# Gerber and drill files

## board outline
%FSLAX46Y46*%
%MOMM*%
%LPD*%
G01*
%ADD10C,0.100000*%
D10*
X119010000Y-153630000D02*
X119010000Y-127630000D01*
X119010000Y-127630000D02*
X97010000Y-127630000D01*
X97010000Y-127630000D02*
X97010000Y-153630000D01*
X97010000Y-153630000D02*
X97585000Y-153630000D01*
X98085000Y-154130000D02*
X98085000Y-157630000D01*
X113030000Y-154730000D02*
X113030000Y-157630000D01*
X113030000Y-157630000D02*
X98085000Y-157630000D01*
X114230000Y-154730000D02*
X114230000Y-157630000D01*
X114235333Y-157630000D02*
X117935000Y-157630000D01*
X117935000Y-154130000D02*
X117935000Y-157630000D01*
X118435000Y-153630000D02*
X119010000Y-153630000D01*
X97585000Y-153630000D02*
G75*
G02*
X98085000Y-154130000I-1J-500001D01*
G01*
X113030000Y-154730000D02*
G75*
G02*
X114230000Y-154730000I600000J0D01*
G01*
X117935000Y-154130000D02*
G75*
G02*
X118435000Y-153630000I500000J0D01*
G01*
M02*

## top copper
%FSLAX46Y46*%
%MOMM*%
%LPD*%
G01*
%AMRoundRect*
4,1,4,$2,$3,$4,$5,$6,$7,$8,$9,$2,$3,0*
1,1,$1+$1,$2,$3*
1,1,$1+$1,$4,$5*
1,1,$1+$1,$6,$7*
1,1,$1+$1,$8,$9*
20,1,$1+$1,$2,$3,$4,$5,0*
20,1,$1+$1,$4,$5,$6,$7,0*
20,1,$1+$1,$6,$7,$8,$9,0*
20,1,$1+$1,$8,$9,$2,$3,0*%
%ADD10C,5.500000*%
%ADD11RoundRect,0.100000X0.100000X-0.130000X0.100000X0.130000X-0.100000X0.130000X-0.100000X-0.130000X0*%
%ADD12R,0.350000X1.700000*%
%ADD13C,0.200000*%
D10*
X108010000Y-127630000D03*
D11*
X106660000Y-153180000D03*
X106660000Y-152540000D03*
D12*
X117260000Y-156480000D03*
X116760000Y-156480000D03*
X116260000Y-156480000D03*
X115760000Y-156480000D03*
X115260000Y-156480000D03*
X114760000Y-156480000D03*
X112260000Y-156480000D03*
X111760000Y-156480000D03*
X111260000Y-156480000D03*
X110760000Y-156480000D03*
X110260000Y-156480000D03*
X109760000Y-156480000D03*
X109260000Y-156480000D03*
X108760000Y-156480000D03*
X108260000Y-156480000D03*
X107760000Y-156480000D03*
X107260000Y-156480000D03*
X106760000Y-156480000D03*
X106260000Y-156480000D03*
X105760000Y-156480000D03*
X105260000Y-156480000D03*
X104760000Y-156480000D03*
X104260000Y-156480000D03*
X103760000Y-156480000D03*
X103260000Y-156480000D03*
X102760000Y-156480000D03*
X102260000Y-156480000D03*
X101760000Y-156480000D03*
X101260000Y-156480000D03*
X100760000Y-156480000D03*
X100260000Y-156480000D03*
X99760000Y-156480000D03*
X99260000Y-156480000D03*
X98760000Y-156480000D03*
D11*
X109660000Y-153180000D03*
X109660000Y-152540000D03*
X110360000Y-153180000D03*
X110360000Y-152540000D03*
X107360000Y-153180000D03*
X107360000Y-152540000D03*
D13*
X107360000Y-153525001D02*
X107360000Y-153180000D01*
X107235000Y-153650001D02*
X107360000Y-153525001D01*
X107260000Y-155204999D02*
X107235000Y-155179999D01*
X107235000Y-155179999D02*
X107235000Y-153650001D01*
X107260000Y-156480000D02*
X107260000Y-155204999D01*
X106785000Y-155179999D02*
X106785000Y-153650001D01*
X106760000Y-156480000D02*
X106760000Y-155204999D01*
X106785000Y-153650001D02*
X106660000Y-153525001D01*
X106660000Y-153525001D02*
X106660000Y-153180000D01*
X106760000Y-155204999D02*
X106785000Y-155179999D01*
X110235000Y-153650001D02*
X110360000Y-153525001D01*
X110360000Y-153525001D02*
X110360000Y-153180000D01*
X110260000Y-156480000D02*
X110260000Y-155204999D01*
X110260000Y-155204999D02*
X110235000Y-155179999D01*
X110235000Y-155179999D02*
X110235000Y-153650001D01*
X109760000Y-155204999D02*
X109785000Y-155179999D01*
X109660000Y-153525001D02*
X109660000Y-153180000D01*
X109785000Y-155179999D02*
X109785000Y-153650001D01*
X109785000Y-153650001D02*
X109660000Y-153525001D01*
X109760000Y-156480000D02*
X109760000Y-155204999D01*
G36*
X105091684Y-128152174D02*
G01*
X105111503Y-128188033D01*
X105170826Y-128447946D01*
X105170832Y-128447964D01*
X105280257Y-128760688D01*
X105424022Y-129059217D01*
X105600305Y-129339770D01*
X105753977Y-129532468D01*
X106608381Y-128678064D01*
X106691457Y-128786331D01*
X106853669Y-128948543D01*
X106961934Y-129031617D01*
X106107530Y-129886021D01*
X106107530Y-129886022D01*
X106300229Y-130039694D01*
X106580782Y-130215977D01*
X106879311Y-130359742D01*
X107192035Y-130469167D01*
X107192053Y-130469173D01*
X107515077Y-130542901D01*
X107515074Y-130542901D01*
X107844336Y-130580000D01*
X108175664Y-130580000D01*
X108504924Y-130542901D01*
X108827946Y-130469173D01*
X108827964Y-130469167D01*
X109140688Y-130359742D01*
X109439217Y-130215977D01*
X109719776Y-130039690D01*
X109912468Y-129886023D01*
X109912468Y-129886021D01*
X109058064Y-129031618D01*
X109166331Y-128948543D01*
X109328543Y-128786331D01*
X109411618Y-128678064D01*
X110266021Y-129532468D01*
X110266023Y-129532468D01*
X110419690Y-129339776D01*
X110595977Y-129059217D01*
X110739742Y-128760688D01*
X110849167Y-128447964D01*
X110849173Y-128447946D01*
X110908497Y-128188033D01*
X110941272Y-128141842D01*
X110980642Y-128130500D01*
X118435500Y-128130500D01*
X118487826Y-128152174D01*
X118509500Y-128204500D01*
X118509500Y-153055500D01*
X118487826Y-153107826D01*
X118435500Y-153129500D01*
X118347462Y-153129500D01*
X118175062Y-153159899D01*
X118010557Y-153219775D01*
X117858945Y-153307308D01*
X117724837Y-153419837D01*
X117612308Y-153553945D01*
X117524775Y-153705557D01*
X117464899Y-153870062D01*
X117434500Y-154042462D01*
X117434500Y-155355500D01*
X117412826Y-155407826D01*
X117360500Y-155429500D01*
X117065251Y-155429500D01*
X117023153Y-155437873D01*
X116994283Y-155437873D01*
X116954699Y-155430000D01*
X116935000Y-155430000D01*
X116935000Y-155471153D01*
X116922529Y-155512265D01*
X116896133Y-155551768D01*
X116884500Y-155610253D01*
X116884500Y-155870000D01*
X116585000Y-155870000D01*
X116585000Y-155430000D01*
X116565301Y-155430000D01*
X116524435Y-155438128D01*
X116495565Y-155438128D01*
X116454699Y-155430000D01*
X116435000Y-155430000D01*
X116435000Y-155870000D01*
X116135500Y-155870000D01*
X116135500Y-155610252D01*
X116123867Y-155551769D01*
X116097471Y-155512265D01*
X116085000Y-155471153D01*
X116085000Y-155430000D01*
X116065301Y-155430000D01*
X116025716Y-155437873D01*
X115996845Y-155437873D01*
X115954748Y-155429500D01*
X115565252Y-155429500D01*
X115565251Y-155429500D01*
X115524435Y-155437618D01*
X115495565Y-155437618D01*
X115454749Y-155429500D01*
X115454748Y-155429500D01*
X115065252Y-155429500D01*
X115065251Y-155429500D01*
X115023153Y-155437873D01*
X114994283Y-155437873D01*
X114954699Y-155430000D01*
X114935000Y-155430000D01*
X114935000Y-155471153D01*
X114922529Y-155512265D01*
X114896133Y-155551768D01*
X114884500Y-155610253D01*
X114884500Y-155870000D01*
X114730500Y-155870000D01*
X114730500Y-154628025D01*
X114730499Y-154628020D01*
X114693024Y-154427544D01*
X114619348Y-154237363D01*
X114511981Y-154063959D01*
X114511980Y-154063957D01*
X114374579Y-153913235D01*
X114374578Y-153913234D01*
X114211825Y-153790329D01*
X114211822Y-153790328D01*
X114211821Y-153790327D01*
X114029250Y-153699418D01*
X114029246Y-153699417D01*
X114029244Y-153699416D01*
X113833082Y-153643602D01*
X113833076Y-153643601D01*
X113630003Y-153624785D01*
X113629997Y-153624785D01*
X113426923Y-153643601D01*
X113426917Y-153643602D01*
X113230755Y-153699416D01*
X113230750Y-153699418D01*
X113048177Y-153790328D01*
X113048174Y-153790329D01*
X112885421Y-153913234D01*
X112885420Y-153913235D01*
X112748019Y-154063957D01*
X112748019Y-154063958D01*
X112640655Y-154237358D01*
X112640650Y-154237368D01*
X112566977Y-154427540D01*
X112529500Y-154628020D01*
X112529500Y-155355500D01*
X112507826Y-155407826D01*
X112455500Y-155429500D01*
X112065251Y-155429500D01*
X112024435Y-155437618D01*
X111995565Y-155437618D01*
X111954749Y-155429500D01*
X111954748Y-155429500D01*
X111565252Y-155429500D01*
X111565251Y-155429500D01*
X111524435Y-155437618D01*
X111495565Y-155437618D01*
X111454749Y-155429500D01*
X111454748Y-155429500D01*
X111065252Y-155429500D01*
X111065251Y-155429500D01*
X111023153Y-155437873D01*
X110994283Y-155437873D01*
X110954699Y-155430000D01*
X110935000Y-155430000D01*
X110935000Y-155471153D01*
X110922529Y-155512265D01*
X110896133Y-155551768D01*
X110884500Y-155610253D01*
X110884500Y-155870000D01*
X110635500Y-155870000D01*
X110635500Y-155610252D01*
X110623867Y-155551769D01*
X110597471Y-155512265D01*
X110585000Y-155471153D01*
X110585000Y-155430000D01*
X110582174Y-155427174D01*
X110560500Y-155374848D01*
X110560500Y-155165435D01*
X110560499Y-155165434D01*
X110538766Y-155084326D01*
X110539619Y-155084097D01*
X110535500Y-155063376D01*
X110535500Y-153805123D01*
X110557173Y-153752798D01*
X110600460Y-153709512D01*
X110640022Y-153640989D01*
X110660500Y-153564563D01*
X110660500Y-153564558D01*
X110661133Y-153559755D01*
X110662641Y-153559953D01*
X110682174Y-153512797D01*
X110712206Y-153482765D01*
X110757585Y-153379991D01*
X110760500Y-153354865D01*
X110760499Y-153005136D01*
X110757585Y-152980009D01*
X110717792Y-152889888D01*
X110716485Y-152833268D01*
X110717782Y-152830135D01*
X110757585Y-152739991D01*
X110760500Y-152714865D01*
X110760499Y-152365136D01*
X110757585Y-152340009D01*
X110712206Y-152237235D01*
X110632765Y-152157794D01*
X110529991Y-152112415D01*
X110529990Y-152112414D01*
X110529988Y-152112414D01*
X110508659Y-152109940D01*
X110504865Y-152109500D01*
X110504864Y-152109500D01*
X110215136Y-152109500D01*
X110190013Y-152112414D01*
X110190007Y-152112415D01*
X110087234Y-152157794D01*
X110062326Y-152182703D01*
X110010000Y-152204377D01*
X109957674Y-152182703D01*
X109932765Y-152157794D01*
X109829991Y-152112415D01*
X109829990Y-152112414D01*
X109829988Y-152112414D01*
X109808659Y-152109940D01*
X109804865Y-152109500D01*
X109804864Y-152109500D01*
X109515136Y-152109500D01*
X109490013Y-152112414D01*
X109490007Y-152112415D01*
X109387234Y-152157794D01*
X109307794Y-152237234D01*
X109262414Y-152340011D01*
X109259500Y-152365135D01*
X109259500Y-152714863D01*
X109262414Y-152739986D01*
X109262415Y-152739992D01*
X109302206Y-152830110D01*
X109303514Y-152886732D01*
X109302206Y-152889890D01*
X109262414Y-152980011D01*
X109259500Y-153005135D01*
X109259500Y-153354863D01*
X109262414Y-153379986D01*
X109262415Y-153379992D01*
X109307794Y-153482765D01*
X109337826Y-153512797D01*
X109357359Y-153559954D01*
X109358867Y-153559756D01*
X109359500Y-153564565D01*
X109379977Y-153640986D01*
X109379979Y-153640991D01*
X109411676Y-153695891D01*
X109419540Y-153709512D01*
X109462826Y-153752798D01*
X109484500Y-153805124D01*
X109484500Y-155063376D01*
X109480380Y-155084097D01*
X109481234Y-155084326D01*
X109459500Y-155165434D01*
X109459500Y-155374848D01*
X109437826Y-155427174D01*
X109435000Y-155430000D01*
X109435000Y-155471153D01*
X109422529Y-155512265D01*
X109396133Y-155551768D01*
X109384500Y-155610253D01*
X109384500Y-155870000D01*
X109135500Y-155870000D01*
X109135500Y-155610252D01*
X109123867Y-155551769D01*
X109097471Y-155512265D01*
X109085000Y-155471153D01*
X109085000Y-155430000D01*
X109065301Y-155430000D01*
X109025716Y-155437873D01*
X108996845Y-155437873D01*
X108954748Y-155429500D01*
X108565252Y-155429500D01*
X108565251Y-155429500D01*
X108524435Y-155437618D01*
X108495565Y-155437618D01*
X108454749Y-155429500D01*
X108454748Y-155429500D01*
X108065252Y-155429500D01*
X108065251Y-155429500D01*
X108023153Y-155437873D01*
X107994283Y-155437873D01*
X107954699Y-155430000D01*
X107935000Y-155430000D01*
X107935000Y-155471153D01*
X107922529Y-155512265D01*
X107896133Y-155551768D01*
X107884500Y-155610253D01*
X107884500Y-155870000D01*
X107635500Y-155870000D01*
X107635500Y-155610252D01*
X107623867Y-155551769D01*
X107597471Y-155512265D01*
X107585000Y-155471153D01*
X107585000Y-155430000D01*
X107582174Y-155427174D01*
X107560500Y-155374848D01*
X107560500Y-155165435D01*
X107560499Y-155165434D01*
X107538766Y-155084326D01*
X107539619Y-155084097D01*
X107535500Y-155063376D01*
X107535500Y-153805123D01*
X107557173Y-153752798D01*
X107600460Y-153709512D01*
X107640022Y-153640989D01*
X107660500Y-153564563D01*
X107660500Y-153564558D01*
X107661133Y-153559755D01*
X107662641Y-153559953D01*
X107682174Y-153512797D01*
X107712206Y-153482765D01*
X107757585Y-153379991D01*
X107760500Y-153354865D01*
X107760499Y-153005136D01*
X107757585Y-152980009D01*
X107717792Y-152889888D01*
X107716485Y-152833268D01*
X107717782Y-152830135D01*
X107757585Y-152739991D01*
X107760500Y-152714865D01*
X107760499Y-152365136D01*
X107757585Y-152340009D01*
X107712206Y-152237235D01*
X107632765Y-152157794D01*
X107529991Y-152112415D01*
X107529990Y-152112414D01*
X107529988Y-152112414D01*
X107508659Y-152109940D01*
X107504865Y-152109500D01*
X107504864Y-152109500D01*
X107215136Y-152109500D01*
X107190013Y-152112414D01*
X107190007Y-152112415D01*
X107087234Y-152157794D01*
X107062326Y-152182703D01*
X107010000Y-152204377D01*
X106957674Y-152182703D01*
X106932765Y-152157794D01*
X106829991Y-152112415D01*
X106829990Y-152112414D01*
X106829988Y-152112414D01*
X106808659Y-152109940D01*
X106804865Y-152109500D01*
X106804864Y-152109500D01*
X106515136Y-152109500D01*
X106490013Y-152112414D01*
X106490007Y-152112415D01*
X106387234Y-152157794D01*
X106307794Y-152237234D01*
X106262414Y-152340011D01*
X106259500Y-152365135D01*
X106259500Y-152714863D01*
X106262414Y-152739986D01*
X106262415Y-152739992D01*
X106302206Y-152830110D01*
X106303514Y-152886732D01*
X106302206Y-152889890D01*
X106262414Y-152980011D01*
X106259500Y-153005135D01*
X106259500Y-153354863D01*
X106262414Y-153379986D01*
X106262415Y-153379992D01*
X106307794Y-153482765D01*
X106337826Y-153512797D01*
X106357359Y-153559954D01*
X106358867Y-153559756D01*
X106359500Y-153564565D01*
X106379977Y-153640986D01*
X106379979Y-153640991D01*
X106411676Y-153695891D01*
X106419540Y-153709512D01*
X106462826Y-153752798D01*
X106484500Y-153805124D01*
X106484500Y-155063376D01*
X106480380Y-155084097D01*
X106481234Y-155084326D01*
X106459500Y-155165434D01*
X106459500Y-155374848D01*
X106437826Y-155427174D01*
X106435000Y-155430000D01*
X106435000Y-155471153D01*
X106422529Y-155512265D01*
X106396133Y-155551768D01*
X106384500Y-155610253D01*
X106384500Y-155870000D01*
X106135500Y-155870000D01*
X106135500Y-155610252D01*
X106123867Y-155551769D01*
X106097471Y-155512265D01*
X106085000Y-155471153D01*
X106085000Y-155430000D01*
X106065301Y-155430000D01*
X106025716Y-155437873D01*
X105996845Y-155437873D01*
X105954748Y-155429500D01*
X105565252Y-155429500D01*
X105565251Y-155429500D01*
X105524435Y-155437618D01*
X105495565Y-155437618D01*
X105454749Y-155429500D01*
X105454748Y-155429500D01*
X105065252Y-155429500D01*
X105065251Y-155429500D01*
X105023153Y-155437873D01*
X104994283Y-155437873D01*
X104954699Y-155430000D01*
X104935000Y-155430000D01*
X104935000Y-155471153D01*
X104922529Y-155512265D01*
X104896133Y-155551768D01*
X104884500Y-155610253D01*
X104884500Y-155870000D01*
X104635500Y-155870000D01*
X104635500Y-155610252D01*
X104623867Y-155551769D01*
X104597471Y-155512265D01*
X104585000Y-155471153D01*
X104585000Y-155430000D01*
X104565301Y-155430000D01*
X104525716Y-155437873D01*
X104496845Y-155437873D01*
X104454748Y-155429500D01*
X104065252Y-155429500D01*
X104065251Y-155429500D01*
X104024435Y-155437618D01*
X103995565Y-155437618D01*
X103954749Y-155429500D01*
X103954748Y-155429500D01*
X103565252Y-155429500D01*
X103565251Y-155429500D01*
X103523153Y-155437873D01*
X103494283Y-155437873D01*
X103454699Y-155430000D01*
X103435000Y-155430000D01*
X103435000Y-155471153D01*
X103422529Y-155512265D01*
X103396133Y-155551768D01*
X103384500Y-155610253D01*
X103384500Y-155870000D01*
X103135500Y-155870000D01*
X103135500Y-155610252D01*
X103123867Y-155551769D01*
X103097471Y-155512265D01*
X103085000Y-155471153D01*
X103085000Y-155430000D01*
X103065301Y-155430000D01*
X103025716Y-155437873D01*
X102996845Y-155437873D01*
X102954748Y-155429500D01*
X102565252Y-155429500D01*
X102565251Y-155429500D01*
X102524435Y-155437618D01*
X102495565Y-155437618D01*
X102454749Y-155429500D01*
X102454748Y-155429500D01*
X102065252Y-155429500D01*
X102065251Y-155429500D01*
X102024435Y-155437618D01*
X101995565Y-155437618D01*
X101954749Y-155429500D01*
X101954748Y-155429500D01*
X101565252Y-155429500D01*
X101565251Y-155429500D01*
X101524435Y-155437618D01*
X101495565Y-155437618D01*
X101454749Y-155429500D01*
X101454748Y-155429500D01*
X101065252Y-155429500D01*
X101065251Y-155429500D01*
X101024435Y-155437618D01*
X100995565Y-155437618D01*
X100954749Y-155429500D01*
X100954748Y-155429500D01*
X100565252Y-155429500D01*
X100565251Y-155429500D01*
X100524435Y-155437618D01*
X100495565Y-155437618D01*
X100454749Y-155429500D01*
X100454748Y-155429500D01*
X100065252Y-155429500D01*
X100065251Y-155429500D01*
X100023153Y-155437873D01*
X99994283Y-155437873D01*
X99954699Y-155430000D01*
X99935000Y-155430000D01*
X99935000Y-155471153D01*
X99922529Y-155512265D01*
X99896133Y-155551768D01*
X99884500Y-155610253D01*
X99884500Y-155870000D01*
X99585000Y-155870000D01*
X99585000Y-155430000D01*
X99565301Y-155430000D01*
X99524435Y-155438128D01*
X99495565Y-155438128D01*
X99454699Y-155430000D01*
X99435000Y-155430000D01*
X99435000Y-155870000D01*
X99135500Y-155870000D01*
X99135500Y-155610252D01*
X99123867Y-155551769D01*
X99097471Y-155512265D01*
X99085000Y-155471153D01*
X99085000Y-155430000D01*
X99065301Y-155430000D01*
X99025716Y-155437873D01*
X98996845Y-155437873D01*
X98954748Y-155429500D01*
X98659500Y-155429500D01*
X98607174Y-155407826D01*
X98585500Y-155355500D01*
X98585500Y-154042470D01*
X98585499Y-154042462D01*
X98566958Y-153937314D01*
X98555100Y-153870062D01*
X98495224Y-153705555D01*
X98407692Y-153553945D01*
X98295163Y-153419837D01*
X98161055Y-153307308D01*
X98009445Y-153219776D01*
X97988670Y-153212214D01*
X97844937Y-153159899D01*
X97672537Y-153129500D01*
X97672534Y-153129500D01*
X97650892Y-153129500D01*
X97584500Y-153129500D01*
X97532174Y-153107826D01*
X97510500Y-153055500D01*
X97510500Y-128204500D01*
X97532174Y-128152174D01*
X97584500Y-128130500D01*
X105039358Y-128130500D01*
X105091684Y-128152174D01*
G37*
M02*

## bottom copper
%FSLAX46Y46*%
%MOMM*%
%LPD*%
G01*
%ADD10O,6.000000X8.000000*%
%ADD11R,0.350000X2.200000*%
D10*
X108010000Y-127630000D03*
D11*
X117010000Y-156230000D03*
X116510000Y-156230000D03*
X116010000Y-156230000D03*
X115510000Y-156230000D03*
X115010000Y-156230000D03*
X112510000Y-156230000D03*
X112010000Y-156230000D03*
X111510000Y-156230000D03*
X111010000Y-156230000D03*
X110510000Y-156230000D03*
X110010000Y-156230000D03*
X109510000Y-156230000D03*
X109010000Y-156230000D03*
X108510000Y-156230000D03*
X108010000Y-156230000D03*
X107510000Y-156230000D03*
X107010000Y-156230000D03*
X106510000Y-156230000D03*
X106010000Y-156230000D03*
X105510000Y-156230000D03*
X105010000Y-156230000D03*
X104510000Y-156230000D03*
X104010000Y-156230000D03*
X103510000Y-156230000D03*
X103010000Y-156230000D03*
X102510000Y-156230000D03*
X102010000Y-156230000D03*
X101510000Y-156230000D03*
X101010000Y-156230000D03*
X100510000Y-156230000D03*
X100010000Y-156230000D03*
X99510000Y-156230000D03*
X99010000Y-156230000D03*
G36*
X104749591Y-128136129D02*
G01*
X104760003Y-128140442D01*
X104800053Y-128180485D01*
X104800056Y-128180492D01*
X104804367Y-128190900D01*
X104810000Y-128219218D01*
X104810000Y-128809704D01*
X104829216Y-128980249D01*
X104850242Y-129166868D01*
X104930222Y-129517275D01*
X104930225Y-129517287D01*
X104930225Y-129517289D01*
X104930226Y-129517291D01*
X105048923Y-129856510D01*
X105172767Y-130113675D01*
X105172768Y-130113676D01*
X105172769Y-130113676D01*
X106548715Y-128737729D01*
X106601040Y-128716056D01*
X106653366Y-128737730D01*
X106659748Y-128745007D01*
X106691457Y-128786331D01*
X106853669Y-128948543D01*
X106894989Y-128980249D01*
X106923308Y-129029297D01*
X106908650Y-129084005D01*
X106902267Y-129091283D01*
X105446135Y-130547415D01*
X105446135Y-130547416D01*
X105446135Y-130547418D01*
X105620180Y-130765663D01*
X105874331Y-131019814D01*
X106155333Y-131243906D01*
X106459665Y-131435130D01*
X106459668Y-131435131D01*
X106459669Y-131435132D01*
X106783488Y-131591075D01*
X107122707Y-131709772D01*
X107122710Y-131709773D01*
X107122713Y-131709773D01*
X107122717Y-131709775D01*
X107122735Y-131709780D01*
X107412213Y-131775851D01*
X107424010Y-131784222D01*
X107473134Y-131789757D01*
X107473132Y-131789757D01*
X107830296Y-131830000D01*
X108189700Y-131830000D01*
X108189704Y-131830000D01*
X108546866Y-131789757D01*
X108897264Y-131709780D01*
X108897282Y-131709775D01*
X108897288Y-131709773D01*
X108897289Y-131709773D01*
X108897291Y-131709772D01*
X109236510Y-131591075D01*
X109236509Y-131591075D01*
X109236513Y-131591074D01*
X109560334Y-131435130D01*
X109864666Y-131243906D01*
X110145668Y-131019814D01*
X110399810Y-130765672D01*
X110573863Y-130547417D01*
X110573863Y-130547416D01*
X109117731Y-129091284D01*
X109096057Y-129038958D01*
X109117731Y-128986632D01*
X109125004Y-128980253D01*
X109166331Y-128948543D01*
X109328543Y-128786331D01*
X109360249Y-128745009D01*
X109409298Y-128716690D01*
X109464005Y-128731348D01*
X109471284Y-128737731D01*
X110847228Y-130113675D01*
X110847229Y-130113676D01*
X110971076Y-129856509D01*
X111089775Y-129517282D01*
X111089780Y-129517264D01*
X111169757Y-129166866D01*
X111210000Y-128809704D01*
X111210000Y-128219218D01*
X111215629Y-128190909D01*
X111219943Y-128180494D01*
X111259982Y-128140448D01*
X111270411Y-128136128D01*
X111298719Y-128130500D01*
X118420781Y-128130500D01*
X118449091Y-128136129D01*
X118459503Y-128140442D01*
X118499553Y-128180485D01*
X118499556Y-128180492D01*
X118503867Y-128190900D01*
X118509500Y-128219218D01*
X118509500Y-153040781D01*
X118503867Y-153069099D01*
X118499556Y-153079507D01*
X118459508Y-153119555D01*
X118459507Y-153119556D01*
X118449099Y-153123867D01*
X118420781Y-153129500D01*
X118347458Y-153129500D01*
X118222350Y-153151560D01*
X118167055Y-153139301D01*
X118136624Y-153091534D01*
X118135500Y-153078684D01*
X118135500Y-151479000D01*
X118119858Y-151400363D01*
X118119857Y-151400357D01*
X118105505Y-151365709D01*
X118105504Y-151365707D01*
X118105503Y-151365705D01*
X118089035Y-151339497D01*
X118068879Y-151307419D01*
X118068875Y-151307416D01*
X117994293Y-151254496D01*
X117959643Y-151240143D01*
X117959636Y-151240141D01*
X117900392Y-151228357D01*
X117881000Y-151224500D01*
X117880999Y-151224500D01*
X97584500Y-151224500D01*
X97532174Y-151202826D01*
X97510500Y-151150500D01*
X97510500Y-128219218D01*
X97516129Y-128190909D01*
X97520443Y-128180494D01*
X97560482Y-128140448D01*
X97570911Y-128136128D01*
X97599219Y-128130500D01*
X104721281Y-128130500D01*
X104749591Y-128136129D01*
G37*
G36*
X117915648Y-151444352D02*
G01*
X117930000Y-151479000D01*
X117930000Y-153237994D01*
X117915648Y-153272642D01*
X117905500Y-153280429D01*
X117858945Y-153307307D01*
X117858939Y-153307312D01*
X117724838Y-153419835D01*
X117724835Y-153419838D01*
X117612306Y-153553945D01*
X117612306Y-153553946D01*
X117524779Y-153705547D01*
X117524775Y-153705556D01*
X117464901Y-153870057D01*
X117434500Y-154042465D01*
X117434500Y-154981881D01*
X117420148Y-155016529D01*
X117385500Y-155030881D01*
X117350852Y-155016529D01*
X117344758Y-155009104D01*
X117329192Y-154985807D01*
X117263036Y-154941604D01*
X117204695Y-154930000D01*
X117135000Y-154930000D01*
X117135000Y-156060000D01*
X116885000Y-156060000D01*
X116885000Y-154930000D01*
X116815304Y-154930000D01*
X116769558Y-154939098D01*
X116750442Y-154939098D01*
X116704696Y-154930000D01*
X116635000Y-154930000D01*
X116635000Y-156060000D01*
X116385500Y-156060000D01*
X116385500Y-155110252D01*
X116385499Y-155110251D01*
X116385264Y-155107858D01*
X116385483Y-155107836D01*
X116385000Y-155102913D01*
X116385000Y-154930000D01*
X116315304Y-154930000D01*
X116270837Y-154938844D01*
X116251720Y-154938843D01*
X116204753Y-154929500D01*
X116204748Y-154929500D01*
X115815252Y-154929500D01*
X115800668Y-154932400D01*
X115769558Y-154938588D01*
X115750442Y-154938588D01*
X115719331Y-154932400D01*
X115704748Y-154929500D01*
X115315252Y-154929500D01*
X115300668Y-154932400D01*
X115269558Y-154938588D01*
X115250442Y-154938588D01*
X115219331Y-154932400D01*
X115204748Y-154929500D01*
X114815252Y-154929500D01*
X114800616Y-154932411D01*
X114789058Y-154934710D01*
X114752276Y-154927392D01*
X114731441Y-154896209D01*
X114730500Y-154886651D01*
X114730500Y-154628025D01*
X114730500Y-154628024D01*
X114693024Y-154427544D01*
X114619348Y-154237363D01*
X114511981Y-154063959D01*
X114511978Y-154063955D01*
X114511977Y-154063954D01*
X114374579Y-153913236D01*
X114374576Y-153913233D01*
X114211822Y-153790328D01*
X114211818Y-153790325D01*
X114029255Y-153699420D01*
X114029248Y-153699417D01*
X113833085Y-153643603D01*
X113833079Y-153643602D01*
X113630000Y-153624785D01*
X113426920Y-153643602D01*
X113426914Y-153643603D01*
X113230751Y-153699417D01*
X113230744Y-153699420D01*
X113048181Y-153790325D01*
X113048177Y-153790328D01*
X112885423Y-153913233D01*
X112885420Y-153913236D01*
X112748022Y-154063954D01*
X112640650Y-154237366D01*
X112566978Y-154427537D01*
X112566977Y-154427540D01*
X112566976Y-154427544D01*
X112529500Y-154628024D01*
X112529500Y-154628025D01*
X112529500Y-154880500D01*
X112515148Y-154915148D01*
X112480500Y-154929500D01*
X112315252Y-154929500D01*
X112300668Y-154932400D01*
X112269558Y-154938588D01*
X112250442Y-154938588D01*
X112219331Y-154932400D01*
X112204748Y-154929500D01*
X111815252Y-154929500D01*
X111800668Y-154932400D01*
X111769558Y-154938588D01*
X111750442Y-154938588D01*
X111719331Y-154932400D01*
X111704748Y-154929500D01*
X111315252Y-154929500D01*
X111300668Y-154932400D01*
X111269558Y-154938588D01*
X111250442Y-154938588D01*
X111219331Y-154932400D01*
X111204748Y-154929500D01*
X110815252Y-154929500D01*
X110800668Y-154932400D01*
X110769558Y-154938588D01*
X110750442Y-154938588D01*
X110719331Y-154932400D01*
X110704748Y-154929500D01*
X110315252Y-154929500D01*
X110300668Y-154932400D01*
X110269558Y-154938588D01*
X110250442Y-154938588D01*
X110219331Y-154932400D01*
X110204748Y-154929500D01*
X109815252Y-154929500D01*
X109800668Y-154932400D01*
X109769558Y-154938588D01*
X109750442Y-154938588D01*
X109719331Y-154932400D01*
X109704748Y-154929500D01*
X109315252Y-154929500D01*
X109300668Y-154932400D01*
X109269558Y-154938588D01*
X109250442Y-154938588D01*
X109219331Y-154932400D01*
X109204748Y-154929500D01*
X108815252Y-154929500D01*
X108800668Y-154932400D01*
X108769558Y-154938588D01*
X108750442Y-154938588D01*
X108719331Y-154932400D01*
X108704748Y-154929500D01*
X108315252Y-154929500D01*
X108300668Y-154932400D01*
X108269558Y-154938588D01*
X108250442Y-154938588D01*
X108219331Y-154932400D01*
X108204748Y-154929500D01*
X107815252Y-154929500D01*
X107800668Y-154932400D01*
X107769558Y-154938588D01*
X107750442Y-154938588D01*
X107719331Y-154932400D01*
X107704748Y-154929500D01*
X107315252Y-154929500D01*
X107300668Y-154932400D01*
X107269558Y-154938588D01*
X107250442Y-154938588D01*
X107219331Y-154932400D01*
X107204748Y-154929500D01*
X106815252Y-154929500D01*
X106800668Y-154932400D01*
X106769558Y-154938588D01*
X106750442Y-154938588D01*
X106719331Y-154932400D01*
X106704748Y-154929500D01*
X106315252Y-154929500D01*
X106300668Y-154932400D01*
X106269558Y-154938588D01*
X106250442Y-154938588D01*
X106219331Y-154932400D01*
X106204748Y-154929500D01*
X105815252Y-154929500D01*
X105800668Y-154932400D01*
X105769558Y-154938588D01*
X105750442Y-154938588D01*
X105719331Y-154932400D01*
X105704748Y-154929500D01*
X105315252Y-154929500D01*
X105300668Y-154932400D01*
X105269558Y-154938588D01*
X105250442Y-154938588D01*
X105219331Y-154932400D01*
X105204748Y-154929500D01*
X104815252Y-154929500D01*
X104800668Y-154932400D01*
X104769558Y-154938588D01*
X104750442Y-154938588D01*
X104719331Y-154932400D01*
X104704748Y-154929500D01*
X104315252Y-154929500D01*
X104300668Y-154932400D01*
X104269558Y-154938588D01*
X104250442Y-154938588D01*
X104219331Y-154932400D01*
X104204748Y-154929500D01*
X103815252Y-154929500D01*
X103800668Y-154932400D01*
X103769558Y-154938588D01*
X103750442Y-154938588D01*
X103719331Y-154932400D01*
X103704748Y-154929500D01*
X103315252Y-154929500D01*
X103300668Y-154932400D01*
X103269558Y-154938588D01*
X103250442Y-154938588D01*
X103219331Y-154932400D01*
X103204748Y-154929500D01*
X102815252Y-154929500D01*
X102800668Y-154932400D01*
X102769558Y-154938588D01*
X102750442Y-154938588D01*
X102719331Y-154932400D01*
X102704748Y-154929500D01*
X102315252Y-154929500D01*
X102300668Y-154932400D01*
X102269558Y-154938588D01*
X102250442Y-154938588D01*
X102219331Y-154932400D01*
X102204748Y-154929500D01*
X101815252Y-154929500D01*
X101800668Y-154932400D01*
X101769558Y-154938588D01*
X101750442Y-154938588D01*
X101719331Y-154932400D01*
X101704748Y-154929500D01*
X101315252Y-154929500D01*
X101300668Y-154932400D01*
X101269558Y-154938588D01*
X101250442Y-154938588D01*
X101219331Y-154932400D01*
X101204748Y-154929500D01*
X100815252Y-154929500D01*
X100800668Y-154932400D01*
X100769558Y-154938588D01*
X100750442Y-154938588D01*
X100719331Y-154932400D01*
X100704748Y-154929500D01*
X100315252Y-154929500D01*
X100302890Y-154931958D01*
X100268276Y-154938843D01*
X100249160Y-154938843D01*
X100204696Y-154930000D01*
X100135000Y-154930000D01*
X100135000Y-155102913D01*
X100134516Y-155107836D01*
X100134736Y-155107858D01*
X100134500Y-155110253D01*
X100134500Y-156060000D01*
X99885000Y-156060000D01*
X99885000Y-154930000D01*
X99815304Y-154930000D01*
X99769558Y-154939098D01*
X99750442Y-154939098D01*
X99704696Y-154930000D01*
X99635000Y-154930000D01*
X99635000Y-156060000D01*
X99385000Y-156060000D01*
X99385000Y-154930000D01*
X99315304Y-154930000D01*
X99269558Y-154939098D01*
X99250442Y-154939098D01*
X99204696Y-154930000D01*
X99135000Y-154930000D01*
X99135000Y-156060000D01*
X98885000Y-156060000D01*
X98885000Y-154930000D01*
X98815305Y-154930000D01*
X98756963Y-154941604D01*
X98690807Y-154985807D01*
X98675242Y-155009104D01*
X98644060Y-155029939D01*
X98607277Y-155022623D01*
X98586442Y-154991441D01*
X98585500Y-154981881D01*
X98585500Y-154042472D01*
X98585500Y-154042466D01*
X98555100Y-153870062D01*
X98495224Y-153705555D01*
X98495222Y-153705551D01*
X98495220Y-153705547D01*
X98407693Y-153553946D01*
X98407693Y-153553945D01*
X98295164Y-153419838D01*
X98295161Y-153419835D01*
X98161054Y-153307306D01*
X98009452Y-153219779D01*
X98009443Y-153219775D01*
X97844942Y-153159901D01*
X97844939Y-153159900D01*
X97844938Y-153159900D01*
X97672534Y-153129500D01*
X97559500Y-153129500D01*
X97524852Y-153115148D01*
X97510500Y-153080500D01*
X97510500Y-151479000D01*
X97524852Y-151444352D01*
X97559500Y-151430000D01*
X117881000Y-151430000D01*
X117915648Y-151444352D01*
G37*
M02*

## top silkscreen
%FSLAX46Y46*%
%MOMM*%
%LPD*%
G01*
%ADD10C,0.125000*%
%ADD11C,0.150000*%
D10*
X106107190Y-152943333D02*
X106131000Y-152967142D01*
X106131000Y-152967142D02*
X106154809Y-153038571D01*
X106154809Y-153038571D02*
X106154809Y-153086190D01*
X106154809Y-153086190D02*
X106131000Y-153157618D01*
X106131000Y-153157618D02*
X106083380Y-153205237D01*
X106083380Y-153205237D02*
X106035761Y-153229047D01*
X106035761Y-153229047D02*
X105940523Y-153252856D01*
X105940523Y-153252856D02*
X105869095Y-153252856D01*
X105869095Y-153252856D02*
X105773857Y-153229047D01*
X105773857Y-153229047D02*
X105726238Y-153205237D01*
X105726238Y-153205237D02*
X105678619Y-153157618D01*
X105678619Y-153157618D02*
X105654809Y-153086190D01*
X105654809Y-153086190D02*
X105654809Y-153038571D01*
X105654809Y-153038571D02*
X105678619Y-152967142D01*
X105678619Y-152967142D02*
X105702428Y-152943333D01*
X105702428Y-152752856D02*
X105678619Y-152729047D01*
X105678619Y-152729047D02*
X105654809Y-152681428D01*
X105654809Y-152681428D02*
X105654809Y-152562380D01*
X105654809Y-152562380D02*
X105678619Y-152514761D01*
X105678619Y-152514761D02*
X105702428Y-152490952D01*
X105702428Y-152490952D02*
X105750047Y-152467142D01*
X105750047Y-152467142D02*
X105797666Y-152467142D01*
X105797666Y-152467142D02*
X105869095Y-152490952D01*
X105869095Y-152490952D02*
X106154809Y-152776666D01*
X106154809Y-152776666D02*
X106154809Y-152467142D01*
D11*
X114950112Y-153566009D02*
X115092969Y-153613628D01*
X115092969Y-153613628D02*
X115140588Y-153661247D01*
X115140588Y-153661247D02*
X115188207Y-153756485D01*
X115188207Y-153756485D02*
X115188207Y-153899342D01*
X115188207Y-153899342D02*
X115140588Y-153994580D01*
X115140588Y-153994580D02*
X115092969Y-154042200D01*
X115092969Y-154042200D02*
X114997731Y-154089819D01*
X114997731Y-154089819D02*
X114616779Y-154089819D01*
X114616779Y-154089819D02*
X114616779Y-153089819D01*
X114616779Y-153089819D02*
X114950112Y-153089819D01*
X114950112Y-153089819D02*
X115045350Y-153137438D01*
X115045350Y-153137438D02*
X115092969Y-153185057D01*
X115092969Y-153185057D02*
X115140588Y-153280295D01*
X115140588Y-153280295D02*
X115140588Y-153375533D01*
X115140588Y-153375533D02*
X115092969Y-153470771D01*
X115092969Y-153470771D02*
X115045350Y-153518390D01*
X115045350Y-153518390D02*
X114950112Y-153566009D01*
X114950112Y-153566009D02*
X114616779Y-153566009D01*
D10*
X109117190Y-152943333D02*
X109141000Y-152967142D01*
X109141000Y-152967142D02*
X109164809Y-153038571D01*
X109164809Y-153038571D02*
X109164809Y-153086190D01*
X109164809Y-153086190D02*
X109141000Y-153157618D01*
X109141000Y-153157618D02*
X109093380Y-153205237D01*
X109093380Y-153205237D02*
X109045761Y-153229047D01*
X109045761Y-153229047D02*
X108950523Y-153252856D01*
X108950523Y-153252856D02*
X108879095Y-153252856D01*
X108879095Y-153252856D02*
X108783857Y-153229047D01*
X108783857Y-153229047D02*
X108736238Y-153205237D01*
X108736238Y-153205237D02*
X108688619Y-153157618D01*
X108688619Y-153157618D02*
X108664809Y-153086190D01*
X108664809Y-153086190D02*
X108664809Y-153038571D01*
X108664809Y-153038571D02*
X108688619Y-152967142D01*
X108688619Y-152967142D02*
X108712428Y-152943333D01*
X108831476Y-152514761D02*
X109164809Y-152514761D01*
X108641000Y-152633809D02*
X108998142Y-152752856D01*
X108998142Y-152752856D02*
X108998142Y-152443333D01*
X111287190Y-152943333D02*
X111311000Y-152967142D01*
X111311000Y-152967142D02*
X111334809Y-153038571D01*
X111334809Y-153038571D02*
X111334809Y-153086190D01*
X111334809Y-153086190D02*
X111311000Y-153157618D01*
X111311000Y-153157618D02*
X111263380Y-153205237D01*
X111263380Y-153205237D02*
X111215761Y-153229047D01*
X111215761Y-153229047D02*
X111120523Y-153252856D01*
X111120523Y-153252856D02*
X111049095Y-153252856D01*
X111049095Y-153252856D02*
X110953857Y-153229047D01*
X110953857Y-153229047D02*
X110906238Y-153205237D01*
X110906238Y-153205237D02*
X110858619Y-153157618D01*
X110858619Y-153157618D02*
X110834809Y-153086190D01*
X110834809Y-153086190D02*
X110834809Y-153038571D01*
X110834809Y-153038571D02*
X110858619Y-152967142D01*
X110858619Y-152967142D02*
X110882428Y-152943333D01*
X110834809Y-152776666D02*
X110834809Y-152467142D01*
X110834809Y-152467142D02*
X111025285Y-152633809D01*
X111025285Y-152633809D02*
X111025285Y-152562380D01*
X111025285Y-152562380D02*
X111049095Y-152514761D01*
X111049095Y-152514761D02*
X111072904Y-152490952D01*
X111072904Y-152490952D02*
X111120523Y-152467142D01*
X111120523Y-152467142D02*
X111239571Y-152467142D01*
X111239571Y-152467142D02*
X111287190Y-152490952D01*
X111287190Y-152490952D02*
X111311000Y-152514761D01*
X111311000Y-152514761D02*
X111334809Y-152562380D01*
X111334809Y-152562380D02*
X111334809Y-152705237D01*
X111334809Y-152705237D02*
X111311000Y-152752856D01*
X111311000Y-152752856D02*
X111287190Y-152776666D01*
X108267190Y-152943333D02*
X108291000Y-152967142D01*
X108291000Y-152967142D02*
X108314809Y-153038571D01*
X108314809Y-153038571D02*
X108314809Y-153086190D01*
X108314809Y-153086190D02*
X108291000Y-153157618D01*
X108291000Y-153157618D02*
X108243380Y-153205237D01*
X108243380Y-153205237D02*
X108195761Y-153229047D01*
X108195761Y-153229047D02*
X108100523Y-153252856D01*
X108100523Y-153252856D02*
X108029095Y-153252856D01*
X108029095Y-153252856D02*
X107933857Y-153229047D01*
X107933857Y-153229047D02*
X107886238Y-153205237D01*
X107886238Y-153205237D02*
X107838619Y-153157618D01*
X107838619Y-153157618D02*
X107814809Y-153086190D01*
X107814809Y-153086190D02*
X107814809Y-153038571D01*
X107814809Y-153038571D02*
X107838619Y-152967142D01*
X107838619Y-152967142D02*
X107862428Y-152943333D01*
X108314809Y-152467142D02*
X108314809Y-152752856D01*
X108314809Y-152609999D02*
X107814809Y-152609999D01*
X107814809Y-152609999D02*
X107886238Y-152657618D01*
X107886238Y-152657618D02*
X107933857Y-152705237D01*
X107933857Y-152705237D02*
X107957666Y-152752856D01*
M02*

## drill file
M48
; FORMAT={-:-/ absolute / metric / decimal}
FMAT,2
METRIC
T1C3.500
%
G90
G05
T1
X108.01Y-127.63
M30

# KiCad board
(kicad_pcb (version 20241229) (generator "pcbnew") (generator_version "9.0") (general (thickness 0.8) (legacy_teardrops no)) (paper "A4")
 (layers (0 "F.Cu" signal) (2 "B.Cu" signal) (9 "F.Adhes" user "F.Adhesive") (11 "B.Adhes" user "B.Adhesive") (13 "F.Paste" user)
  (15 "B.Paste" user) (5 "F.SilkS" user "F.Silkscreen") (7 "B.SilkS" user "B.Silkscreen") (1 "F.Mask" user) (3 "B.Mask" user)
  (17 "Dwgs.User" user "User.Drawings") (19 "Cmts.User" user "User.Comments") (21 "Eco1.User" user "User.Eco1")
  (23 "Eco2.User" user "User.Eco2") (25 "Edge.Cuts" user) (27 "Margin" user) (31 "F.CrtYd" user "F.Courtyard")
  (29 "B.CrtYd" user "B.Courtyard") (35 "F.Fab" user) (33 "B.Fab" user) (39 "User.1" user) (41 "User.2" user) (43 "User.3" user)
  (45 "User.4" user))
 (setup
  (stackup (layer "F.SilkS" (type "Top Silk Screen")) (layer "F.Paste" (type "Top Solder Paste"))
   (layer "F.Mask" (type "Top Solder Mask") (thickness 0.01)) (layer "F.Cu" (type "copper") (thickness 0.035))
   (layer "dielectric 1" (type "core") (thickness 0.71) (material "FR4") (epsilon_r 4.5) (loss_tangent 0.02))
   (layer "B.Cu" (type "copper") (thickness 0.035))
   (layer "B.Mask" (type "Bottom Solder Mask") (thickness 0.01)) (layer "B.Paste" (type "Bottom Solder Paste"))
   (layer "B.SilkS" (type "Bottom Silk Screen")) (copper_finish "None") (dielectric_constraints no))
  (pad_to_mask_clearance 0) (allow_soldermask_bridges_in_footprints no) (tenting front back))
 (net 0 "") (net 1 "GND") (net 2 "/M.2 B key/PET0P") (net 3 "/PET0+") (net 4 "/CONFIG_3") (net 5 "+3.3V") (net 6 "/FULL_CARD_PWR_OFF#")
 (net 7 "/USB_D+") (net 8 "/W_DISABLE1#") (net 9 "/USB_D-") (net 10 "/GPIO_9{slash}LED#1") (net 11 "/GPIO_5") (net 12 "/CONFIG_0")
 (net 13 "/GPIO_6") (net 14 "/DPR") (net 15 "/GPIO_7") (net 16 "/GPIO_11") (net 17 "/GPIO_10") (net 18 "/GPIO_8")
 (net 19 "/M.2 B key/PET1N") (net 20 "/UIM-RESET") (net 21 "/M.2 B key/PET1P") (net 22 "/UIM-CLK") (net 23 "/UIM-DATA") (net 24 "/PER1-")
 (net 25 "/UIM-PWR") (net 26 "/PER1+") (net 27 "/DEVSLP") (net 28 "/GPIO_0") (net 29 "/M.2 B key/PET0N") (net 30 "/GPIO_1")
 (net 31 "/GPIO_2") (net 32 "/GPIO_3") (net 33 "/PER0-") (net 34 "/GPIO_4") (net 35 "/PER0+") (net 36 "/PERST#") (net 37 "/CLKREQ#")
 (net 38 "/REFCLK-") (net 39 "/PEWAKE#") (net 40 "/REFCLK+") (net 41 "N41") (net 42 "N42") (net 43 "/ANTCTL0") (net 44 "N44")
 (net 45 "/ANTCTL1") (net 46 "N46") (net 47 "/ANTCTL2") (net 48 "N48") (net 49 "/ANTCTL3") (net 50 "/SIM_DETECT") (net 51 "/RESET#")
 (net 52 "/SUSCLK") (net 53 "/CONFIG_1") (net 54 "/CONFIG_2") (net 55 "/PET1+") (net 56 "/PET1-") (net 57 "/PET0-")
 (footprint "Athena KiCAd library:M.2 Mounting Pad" (layer "F.Cu") (at 108.01 127.63)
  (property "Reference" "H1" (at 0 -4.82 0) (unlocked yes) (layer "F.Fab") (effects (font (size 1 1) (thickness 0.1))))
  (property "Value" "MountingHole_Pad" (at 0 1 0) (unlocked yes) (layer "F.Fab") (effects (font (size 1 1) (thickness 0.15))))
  (pad "1" thru_hole circle (at 0 0) (size 5.5 5.5) (drill 3.5) (layers "*.Cu" "*.Mask") (remove_unused_layers no) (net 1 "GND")
   (padstack (mode front_inner_back)
    (layer "Inner" (shape circle) (size 5.5 5.5) (zone_connect -1))
    (layer "B.Cu" (shape oval) (size 6 8) (thermal_bridge_angle 45) (zone_connect -1)))))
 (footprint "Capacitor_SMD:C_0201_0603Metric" (layer "F.Cu") (at 106.66 152.86 90)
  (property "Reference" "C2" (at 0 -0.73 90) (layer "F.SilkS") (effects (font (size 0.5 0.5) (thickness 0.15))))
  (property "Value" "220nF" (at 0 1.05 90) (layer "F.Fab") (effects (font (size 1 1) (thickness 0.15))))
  (pad "" smd roundrect (at -0.345 0 90) (size 0.318 0.36) (layers "F.Paste") (roundrect_rratio 0.25))
  (pad "" smd roundrect (at 0.345 0 90) (size 0.318 0.36) (layers "F.Paste") (roundrect_rratio 0.25))
  (pad "1" smd roundrect (at -0.32 0 90) (size 0.46 0.4) (layers "F.Cu" "F.Mask") (roundrect_rratio 0.25) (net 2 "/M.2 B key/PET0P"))
  (pad "2" smd roundrect (at 0.32 0 90) (size 0.46 0.4) (layers "F.Cu" "F.Mask") (roundrect_rratio 0.25) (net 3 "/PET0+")))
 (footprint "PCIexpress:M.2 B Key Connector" (layer "F.Cu") (at 108.01 156.52)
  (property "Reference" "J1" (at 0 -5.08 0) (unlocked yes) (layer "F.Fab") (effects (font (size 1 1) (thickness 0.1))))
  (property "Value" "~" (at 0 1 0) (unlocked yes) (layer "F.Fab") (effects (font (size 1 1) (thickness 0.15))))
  (fp_line (start -11 -2.89) (end -10.425 -2.89) (stroke (width 0.1) (type default)) (layer "Edge.Cuts"))
  (fp_line (start -9.925 -2.39) (end -9.925 1.11) (stroke (width 0.1) (type default)) (layer "Edge.Cuts"))
  (fp_line (start 5.02 -1.79) (end 5.02 1.11) (stroke (width 0.1) (type default)) (layer "Edge.Cuts"))
  (fp_line (start 5.02 1.11) (end -9.925 1.11) (stroke (width 0.1) (type default)) (layer "Edge.Cuts"))
  (fp_line (start 6.22 -1.79) (end 6.22 1.11) (stroke (width 0.1) (type default)) (layer "Edge.Cuts"))
  (fp_line (start 6.225333 1.11) (end 9.925 1.11) (stroke (width 0.1) (type default)) (layer "Edge.Cuts"))
  (fp_line (start 9.925 -2.39) (end 9.925 1.11) (stroke (width 0.1) (type default)) (layer "Edge.Cuts"))
  (fp_line (start 10.425 -2.89) (end 11 -2.89) (stroke (width 0.1) (type default)) (layer "Edge.Cuts"))
  (fp_arc (start -10.425 -2.89) (mid -10.071447 -2.743553) (end -9.925 -2.39) (stroke (width 0.1) (type default)) (layer "Edge.Cuts"))
  (fp_arc (start 5.02 -1.79) (mid 5.62 -2.39) (end 6.22 -1.79) (stroke (width 0.1) (type default)) (layer "Edge.Cuts"))
  (fp_arc (start 9.925 -2.39) (mid 10.071447 -2.743553) (end 10.425 -2.89) (stroke (width 0.1) (type default)) (layer "Edge.Cuts"))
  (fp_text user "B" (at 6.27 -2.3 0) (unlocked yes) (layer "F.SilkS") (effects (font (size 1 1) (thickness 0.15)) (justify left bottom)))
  (pad "1" smd rect (at 9.25 -0.04 180) (size 0.35 1.7) (layers "F.Cu") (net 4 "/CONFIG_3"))
  (pad "2" smd rect (at 9 -0.29 180) (size 0.35 2.2) (layers "B.Cu") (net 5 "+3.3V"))
  (pad "3" smd rect (at 8.75 -0.04 180) (size 0.35 1.7) (layers "F.Cu") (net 1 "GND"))
  (pad "4" smd rect (at 8.5 -0.29 180) (size 0.35 2.2) (layers "B.Cu") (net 5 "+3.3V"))
  (pad "5" smd rect (at 8.25 -0.04 180) (size 0.35 1.7) (layers "F.Cu") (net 1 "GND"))
  (pad "6" smd rect (at 8 -0.29 180) (size 0.35 2.2) (layers "B.Cu") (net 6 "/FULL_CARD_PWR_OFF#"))
  (pad "7" smd rect (at 7.75 -0.04 180) (size 0.35 1.7) (layers "F.Cu") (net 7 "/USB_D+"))
  (pad "8" smd rect (at 7.5 -0.29 180) (size 0.35 2.2) (layers "B.Cu") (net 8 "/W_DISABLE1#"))
  (pad "9" smd rect (at 7.25 -0.04 180) (size 0.35 1.7) (layers "F.Cu") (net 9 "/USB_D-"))
  (pad "10" smd rect (at 7 -0.29 180) (size 0.35 2.2) (layers "B.Cu") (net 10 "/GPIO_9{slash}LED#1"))
  (pad "11" smd rect (at 6.75 -0.04 180) (size 0.35 1.7) (layers "F.Cu") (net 1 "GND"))
  (pad "20" smd rect (at 4.5 -0.29 180) (size 0.35 2.2) (layers "B.Cu") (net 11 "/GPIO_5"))
  (pad "21" smd rect (at 4.25 -0.04 180) (size 0.35 1.7) (layers "F.Cu") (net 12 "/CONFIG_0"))
  (pad "22" smd rect (at 4 -0.29 180) (size 0.35 2.2) (layers "B.Cu") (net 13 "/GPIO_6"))
  (pad "23" smd rect (at 3.75 -0.04 180) (size 0.35 1.7) (layers "F.Cu") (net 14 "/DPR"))
  (pad "24" smd rect (at 3.5 -0.29 180) (size 0.35 2.2) (layers "B.Cu") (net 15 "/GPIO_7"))
  (pad "25" smd rect (at 3.25 -0.04 180) (size 0.35 1.7) (layers "F.Cu") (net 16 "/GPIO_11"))
  (pad "26" smd rect (at 3 -0.29 180) (size 0.35 2.2) (layers "B.Cu") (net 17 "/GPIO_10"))
  (pad "27" smd rect (at 2.75 -0.04 180) (size 0.35 1.7) (layers "F.Cu") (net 1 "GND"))
  (pad "28" smd rect (at 2.5 -0.29 180) (size 0.35 2.2) (layers "B.Cu") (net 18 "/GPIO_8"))
  (pad "29" smd rect (at 2.25 -0.04 180) (size 0.35 1.7) (layers "F.Cu") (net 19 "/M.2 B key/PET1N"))
  (pad "30" smd rect (at 2 -0.29 180) (size 0.35 2.2) (layers "B.Cu") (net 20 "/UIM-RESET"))
  (pad "31" smd rect (at 1.75 -0.04 180) (size 0.35 1.7) (layers "F.Cu") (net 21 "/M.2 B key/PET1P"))
  (pad "32" smd rect (at 1.5 -0.29 180) (size 0.35 2.2) (layers "B.Cu") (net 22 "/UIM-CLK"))
  (pad "33" smd rect (at 1.25 -0.04 180) (size 0.35 1.7) (layers "F.Cu") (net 1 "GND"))
  (pad "34" smd rect (at 1 -0.29 180) (size 0.35 2.2) (layers "B.Cu") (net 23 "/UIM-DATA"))
  (pad "35" smd rect (at 0.75 -0.04 180) (size 0.35 1.7) (layers "F.Cu") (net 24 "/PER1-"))
  (pad "36" smd rect (at 0.5 -0.29 180) (size 0.35 2.2) (layers "B.Cu") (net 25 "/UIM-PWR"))
  (pad "37" smd rect (at 0.25 -0.04 180) (size 0.35 1.7) (layers "F.Cu") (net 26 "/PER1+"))
  (pad "38" smd rect (at 0 -0.29 180) (size 0.35 2.2) (layers "B.Cu") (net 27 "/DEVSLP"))
  (pad "39" smd rect (at -0.25 -0.04 180) (size 0.35 1.7) (layers "F.Cu") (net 1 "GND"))
  (pad "40" smd rect (at -0.5 -0.29 180) (size 0.35 2.2) (layers "B.Cu") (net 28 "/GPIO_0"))
  (pad "41" smd rect (at -0.75 -0.04 180) (size 0.35 1.7) (layers "F.Cu") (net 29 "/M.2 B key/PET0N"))
  (pad "42" smd rect (at -1 -0.29 180) (size 0.35 2.2) (layers "B.Cu") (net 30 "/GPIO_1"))
  (pad "43" smd rect (at -1.25 -0.04 180) (size 0.35 1.7) (layers "F.Cu") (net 2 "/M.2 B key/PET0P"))
  (pad "44" smd rect (at -1.5 -0.29 180) (size 0.35 2.2) (layers "B.Cu") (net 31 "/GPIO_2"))
  (pad "45" smd rect (at -1.75 -0.04 180) (size 0.35 1.7) (layers "F.Cu") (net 1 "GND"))
  (pad "46" smd rect (at -2 -0.29 180) (size 0.35 2.2) (layers "B.Cu") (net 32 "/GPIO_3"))
  (pad "47" smd rect (at -2.25 -0.04 180) (size 0.35 1.7) (layers "F.Cu") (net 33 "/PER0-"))
  (pad "48" smd rect (at -2.5 -0.29 180) (size 0.35 2.2) (layers "B.Cu") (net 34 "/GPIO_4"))
  (pad "49" smd rect (at -2.75 -0.04 180) (size 0.35 1.7) (layers "F.Cu") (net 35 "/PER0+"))
  (pad "50" smd rect (at -3 -0.29 180) (size 0.35 2.2) (layers "B.Cu") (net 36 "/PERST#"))
  (pad "51" smd rect (at -3.25 -0.04 180) (size 0.35 1.7) (layers "F.Cu") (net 1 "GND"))
  (pad "52" smd rect (at -3.5 -0.29 180) (size 0.35 2.2) (layers "B.Cu") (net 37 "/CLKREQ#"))
  (pad "53" smd rect (at -3.75 -0.04 180) (size 0.35 1.7) (layers "F.Cu") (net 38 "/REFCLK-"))
  (pad "54" smd rect (at -4 -0.29 180) (size 0.35 2.2) (layers "B.Cu") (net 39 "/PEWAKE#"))
  (pad "55" smd rect (at -4.25 -0.04 180) (size 0.35 1.7) (layers "F.Cu") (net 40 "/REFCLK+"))
  (pad "56" smd rect (at -4.5 -0.29 180) (size 0.35 2.2) (layers "B.Cu") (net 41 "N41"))
  (pad "57" smd rect (at -4.75 -0.04 180) (size 0.35 1.7) (layers "F.Cu") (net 1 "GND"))
  (pad "58" smd rect (at -5 -0.29 180) (size 0.35 2.2) (layers "B.Cu") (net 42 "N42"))
  (pad "59" smd rect (at -5.25 -0.04 180) (size 0.35 1.7) (layers "F.Cu") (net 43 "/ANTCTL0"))
  (pad "60" smd rect (at -5.5 -0.29 180) (size 0.35 2.2) (layers "B.Cu") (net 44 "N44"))
  (pad "61" smd rect (at -5.75 -0.04 180) (size 0.35 1.7) (layers "F.Cu") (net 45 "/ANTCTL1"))
  (pad "62" smd rect (at -6 -0.29 180) (size 0.35 2.2) (layers "B.Cu") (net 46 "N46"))
  (pad "63" smd rect (at -6.25 -0.04 180) (size 0.35 1.7) (layers "F.Cu") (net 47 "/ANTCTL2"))
  (pad "64" smd rect (at -6.5 -0.29 180) (size 0.35 2.2) (layers "B.Cu") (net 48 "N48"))
  (pad "65" smd rect (at -6.75 -0.04 180) (size 0.35 1.7) (layers "F.Cu") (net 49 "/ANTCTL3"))
  (pad "66" smd rect (at -7 -0.29 180) (size 0.35 2.2) (layers "B.Cu") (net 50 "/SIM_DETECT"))
  (pad "67" smd rect (at -7.25 -0.04 180) (size 0.35 1.7) (layers "F.Cu") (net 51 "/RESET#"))
  (pad "68" smd rect (at -7.5 -0.29 180) (size 0.35 2.2) (layers "B.Cu") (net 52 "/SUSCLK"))
  (pad "69" smd rect (at -7.75 -0.04 180) (size 0.35 1.7) (layers "F.Cu") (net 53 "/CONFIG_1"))
  (pad "70" smd rect (at -8 -0.29 180) (size 0.35 2.2) (layers "B.Cu") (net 5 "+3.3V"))
  (pad "71" smd rect (at -8.25 -0.04 180) (size 0.35 1.7) (layers "F.Cu") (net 1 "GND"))
  (pad "72" smd rect (at -8.5 -0.29 180) (size 0.35 2.2) (layers "B.Cu") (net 5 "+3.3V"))
  (pad "73" smd rect (at -8.75 -0.04 180) (size 0.35 1.7) (layers "F.Cu") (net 1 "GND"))
  (pad "74" smd rect (at -9 -0.29 180) (size 0.35 2.2) (layers "B.Cu") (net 5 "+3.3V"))
  (pad "75" smd rect (at -9.25 -0.04 180) (size 0.35 1.7) (layers "F.Cu") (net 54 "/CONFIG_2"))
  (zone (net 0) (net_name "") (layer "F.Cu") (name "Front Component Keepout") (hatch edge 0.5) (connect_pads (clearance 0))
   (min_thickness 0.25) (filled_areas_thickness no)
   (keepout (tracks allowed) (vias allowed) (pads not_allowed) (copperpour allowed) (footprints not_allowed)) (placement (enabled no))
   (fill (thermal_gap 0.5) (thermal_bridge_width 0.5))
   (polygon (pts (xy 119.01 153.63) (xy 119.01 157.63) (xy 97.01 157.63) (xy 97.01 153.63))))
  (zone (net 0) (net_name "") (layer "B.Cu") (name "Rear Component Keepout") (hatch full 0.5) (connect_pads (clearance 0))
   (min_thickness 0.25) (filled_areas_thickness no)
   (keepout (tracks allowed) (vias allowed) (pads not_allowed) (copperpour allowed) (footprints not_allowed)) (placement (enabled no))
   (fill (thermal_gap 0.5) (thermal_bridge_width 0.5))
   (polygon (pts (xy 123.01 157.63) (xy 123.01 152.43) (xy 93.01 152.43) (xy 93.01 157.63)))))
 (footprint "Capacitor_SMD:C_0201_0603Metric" (layer "F.Cu") (at 109.66 152.86 90)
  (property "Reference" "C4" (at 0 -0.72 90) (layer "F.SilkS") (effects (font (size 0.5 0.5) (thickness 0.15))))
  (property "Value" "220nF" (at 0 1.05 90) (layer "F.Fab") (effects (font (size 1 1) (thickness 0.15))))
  (pad "" smd roundrect (at -0.345 0 90) (size 0.318 0.36) (layers "F.Paste") (roundrect_rratio 0.25))
  (pad "" smd roundrect (at 0.345 0 90) (size 0.318 0.36) (layers "F.Paste") (roundrect_rratio 0.25))
  (pad "1" smd roundrect (at -0.32 0 90) (size 0.46 0.4) (layers "F.Cu" "F.Mask") (roundrect_rratio 0.25) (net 21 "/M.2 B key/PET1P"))
  (pad "2" smd roundrect (at 0.32 0 90) (size 0.46 0.4) (layers "F.Cu" "F.Mask") (roundrect_rratio 0.25) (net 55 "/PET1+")))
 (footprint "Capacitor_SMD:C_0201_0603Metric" (layer "F.Cu") (at 110.36 152.86 90)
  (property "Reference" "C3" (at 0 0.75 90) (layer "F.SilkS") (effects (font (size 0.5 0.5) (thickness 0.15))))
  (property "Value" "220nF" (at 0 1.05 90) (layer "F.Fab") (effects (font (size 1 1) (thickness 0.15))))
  (pad "" smd roundrect (at -0.345 0 90) (size 0.318 0.36) (layers "F.Paste") (roundrect_rratio 0.25))
  (pad "" smd roundrect (at 0.345 0 90) (size 0.318 0.36) (layers "F.Paste") (roundrect_rratio 0.25))
  (pad "1" smd roundrect (at -0.32 0 90) (size 0.46 0.4) (layers "F.Cu" "F.Mask") (roundrect_rratio 0.25) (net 19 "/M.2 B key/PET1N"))
  (pad "2" smd roundrect (at 0.32 0 90) (size 0.46 0.4) (layers "F.Cu" "F.Mask") (roundrect_rratio 0.25) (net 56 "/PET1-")))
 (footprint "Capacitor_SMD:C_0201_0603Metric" (layer "F.Cu") (at 107.36 152.86 90)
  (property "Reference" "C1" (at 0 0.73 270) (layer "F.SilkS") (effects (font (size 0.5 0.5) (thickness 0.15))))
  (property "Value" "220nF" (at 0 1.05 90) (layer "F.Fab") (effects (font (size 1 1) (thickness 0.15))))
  (pad "" smd roundrect (at -0.345 0 90) (size 0.318 0.36) (layers "F.Paste") (roundrect_rratio 0.25))
  (pad "" smd roundrect (at 0.345 0 90) (size 0.318 0.36) (layers "F.Paste") (roundrect_rratio 0.25))
  (pad "1" smd roundrect (at -0.32 0 90) (size 0.46 0.4) (layers "F.Cu" "F.Mask") (roundrect_rratio 0.25) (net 29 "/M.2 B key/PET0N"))
  (pad "2" smd roundrect (at 0.32 0 90) (size 0.46 0.4) (layers "F.Cu" "F.Mask") (roundrect_rratio 0.25) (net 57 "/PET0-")))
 (gr_line (start 119.01 153.63) (end 119.01 127.63) (stroke (width 0.1) (type default)) (layer "Edge.Cuts"))
 (gr_line (start 119.01 127.63) (end 97.01 127.63) (stroke (width 0.1) (type default)) (layer "Edge.Cuts"))
 (gr_line (start 97.01 127.63) (end 97.01 153.63) (stroke (width 0.1) (type default)) (layer "Edge.Cuts"))
 (segment (start 107.36 153.525001) (end 107.36 153.18) (width 0.2) (layer "F.Cu") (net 29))
 (segment (start 107.235 153.650001) (end 107.36 153.525001) (width 0.2) (layer "F.Cu") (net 29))
 (segment (start 107.26 155.204999) (end 107.235 155.179999) (width 0.2) (layer "F.Cu") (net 29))
 (segment (start 107.235 155.179999) (end 107.235 153.650001) (width 0.2) (layer "F.Cu") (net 29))
 (segment (start 107.26 156.48) (end 107.26 155.204999) (width 0.2) (layer "F.Cu") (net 29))
 (segment (start 106.785 155.179999) (end 106.785 153.650001) (width 0.2) (layer "F.Cu") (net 2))
 (segment (start 106.76 156.48) (end 106.76 155.204999) (width 0.2) (layer "F.Cu") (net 2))
 (segment (start 106.785 153.650001) (end 106.66 153.525001) (width 0.2) (layer "F.Cu") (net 2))
 (segment (start 106.66 153.525001) (end 106.66 153.18) (width 0.2) (layer "F.Cu") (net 2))
 (segment (start 106.76 155.204999) (end 106.785 155.179999) (width 0.2) (layer "F.Cu") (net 2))
 (segment (start 110.235 153.650001) (end 110.36 153.525001) (width 0.2) (layer "F.Cu") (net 19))
 (segment (start 110.36 153.525001) (end 110.36 153.18) (width 0.2) (layer "F.Cu") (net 19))
 (segment (start 110.26 156.48) (end 110.26 155.204999) (width 0.2) (layer "F.Cu") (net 19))
 (segment (start 110.26 155.204999) (end 110.235 155.179999) (width 0.2) (layer "F.Cu") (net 19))
 (segment (start 110.235 155.179999) (end 110.235 153.650001) (width 0.2) (layer "F.Cu") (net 19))
 (segment (start 109.76 155.204999) (end 109.785 155.179999) (width 0.2) (layer "F.Cu") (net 21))
 (segment (start 109.66 153.525001) (end 109.66 153.18) (width 0.2) (layer "F.Cu") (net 21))
 (segment (start 109.785 155.179999) (end 109.785 153.650001) (width 0.2) (layer "F.Cu") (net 21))
 (segment (start 109.785 153.650001) (end 109.66 153.525001) (width 0.2) (layer "F.Cu") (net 21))
 (segment (start 109.76 156.48) (end 109.76 155.204999) (width 0.2) (layer "F.Cu") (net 21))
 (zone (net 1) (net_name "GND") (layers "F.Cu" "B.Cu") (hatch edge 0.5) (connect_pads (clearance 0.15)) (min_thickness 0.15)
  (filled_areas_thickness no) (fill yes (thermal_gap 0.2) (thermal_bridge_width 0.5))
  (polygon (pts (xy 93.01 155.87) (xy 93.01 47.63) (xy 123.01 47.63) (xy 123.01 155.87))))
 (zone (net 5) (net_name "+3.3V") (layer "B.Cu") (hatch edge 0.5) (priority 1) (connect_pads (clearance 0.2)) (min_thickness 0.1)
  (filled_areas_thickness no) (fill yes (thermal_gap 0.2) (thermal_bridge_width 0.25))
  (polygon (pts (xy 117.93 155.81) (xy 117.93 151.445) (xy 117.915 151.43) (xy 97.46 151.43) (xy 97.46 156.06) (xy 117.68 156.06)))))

